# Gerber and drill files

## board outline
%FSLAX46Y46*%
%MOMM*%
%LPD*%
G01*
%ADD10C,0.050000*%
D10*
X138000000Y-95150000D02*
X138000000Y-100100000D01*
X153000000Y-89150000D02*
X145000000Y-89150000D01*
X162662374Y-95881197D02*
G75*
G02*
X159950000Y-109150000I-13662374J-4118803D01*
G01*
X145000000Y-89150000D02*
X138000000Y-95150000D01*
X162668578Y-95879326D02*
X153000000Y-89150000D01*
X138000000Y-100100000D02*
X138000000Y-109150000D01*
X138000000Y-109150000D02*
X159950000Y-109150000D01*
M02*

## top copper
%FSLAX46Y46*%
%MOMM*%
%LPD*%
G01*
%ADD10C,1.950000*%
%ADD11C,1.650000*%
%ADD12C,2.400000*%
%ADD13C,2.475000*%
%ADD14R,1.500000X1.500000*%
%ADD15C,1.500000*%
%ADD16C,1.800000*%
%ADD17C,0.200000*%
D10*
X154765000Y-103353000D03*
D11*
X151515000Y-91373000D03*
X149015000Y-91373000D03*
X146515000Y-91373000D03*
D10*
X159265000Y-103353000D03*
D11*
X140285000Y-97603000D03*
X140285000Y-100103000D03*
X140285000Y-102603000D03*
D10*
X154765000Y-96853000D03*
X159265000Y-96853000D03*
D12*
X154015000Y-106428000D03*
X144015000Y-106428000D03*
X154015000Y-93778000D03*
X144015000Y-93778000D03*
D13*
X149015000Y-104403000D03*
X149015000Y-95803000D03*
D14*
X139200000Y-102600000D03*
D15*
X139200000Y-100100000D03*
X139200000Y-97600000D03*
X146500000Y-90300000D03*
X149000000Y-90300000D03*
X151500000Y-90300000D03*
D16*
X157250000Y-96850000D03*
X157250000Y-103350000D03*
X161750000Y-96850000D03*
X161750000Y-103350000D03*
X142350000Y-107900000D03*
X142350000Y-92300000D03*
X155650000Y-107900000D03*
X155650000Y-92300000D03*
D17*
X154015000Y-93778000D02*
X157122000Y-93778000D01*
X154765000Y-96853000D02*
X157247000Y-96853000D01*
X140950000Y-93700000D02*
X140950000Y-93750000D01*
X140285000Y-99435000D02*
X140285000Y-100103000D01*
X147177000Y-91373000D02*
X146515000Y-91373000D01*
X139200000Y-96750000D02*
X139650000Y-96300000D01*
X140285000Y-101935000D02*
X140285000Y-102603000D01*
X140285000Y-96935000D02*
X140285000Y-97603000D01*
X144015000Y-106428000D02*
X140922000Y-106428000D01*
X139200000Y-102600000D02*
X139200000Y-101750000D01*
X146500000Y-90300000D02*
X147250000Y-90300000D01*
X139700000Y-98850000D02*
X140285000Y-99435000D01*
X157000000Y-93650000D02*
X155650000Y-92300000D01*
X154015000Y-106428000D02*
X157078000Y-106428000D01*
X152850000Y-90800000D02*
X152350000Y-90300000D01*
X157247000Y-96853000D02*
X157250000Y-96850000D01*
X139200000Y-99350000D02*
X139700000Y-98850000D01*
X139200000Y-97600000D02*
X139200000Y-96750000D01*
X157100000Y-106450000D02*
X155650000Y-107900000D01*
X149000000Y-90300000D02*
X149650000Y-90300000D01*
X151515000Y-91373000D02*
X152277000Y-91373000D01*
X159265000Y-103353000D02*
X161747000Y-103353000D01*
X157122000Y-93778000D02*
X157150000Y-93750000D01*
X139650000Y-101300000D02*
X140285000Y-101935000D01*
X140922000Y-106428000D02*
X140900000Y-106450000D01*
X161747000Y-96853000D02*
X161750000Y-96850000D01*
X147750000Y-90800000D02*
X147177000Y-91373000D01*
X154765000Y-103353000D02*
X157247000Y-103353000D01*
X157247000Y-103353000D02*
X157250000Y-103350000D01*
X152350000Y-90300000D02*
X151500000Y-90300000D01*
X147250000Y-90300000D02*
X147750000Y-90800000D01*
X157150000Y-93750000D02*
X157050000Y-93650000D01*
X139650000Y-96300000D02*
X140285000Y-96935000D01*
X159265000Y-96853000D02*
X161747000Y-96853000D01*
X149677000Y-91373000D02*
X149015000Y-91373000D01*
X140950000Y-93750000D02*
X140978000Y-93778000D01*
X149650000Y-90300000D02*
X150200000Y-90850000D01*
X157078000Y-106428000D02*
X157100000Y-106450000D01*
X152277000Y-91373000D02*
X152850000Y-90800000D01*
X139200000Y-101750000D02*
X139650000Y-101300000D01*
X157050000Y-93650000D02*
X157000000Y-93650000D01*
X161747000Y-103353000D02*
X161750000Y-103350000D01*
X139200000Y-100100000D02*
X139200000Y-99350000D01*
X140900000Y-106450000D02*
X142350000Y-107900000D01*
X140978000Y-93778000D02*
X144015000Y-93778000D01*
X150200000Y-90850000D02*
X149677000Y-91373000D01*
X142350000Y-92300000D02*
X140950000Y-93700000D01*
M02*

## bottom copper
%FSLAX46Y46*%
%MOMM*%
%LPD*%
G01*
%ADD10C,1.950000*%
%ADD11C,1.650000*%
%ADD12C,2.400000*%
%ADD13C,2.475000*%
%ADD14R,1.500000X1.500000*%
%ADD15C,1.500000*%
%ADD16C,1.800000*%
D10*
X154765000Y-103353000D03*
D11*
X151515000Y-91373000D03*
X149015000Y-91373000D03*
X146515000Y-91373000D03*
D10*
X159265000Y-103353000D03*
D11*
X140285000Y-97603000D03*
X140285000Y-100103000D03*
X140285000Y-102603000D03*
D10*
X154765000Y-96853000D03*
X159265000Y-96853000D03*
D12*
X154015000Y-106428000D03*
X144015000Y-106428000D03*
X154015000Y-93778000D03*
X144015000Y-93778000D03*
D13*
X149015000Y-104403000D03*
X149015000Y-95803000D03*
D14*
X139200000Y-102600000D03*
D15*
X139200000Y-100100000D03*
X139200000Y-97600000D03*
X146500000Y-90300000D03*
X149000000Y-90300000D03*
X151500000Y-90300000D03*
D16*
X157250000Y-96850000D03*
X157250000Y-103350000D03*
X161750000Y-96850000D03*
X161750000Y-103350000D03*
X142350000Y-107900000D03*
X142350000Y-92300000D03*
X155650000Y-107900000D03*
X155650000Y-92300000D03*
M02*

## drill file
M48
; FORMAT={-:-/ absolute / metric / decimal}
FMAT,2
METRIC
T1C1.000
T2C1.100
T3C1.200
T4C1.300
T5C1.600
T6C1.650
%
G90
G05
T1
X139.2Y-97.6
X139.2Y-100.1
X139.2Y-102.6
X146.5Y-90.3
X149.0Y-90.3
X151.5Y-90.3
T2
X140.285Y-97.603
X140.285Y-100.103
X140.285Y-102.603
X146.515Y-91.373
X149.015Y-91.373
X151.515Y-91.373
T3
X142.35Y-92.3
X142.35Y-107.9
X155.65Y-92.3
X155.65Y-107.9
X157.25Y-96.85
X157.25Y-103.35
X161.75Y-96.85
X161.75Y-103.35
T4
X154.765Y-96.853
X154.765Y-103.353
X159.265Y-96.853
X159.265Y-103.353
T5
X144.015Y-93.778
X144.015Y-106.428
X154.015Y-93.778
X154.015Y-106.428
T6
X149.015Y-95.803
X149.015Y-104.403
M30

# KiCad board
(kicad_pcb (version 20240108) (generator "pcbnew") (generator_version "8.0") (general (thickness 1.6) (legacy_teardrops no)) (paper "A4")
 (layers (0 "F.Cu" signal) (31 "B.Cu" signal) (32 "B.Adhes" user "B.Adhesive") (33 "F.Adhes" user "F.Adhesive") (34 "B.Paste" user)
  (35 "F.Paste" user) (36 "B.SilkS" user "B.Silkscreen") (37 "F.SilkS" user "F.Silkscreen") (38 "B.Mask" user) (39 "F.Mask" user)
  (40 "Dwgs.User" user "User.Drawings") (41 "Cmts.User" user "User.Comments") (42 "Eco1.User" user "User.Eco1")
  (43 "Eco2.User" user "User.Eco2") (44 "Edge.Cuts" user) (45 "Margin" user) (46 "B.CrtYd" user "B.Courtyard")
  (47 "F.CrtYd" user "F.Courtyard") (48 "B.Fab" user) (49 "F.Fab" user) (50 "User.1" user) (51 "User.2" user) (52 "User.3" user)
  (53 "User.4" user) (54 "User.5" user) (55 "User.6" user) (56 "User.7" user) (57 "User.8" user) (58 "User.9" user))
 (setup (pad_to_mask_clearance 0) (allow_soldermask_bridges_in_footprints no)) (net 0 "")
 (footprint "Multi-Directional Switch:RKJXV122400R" (layer "F.Cu") (at 149.2 98.5)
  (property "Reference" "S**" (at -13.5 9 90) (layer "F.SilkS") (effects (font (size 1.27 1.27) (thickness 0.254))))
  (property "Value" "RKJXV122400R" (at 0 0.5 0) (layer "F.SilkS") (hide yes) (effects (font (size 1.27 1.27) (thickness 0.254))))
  (pad "A1" thru_hole circle (at 5.565 4.853 90) (size 1.95 1.95) (drill 1.3) (layers "*.Cu" "*.Mask") (remove_unused_layers no))
  (pad "A11" thru_hole circle (at 2.315 -7.127 90) (size 1.65 1.65) (drill 1.1) (layers "*.Cu" "*.Mask") (remove_unused_layers no))
  (pad "A12" thru_hole circle (at -0.185 -7.127 90) (size 1.65 1.65) (drill 1.1) (layers "*.Cu" "*.Mask") (remove_unused_layers no))
  (pad "A13" thru_hole circle (at -2.685 -7.127 90) (size 1.65 1.65) (drill 1.1) (layers "*.Cu" "*.Mask") (remove_unused_layers no))
  (pad "B1" thru_hole circle (at 10.065 4.853 90) (size 1.95 1.95) (drill 1.3) (layers "*.Cu" "*.Mask") (remove_unused_layers no))
  (pad "B11" thru_hole circle (at -8.915 -0.897 90) (size 1.65 1.65) (drill 1.1) (layers "*.Cu" "*.Mask") (remove_unused_layers no))
  (pad "B12" thru_hole circle (at -8.915 1.603 90) (size 1.65 1.65) (drill 1.1) (layers "*.Cu" "*.Mask") (remove_unused_layers no))
  (pad "B13" thru_hole circle (at -8.915 4.103 90) (size 1.65 1.65) (drill 1.1) (layers "*.Cu" "*.Mask") (remove_unused_layers no))
  (pad "C1" thru_hole circle (at 5.565 -1.647 90) (size 1.95 1.95) (drill 1.3) (layers "*.Cu" "*.Mask") (remove_unused_layers no))
  (pad "D1" thru_hole circle (at 10.065 -1.647 90) (size 1.95 1.95) (drill 1.3) (layers "*.Cu" "*.Mask") (remove_unused_layers no))
  (pad "MH1" thru_hole circle (at 4.815 7.928 90) (size 2.4 2.4) (drill 1.6) (layers "*.Cu" "*.Mask") (remove_unused_layers no))
  (pad "MH2" thru_hole circle (at -5.185 7.928 90) (size 2.4 2.4) (drill 1.6) (layers "*.Cu" "*.Mask") (remove_unused_layers no))
  (pad "MH3" thru_hole circle (at 4.815 -4.722 90) (size 2.4 2.4) (drill 1.6) (layers "*.Cu" "*.Mask") (remove_unused_layers no))
  (pad "MH4" thru_hole circle (at -5.185 -4.722 90) (size 2.4 2.4) (drill 1.6) (layers "*.Cu" "*.Mask") (remove_unused_layers no))
  (pad "MH5" thru_hole circle (at -0.185 5.903 90) (size 2.475 2.475) (drill 1.65) (layers "*.Cu" "*.Mask") (remove_unused_layers no))
  (pad "MH6" thru_hole circle (at -0.185 -2.697 90) (size 2.475 2.475) (drill 1.65) (layers "*.Cu" "*.Mask") (remove_unused_layers no)))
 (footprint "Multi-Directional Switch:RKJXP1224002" (layer "F.Cu") (at 150 100)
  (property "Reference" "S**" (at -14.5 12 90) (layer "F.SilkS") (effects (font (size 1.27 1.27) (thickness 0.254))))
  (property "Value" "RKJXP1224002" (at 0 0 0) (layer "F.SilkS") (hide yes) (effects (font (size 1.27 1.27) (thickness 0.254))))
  (pad "1" thru_hole rect (at -10.8 2.6 90) (size 1.5 1.5) (drill 1) (layers "*.Cu" "*.Mask") (remove_unused_layers no))
  (pad "2" thru_hole circle (at -10.8 0.1 90) (size 1.5 1.5) (drill 1) (layers "*.Cu" "*.Mask") (remove_unused_layers no))
  (pad "3" thru_hole circle (at -10.8 -2.4 90) (size 1.5 1.5) (drill 1) (layers "*.Cu" "*.Mask") (remove_unused_layers no))
  (pad "4" thru_hole circle (at -3.5 -9.7 90) (size 1.5 1.5) (drill 1) (layers "*.Cu" "*.Mask") (remove_unused_layers no))
  (pad "5" thru_hole circle (at -1 -9.7 90) (size 1.5 1.5) (drill 1) (layers "*.Cu" "*.Mask") (remove_unused_layers no))
  (pad "6" thru_hole circle (at 1.5 -9.7 90) (size 1.5 1.5) (drill 1) (layers "*.Cu" "*.Mask") (remove_unused_layers no))
  (pad "7" thru_hole circle (at 7.25 -3.15 90) (size 1.8 1.8) (drill 1.2) (layers "*.Cu" "*.Mask") (remove_unused_layers no))
  (pad "8" thru_hole circle (at 7.25 3.35 90) (size 1.8 1.8) (drill 1.2) (layers "*.Cu" "*.Mask") (remove_unused_layers no))
  (pad "9" thru_hole circle (at 11.75 -3.15 90) (size 1.8 1.8) (drill 1.2) (layers "*.Cu" "*.Mask") (remove_unused_layers no))
  (pad "10" thru_hole circle (at 11.75 3.35 90) (size 1.8 1.8) (drill 1.2) (layers "*.Cu" "*.Mask") (remove_unused_layers no))
  (pad "MH1" thru_hole circle (at -7.65 7.9 90) (size 1.8 1.8) (drill 1.2) (layers "*.Cu" "*.Mask") (remove_unused_layers no))
  (pad "MH2" thru_hole circle (at -7.65 -7.7 90) (size 1.8 1.8) (drill 1.2) (layers "*.Cu" "*.Mask") (remove_unused_layers no))
  (pad "MH3" thru_hole circle (at 5.65 7.9 90) (size 1.8 1.8) (drill 1.2) (layers "*.Cu" "*.Mask") (remove_unused_layers no))
  (pad "MH4" thru_hole circle (at 5.65 -7.7 90) (size 1.8 1.8) (drill 1.2) (layers "*.Cu" "*.Mask") (remove_unused_layers no)))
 (gr_line (start 138 95.15) (end 138 100.1) (stroke (width 0.05) (type default)) (layer "Edge.Cuts"))
 (gr_line (start 153 89.15) (end 145 89.15) (stroke (width 0.05) (type default)) (layer "Edge.Cuts"))
 (gr_arc (start 162.662374 95.881197) (mid 162.980612 102.85788) (end 159.95 109.15) (stroke (width 0.05) (type default))
  (layer "Edge.Cuts"))
 (gr_line (start 145 89.15) (end 138 95.15) (stroke (width 0.05) (type default)) (layer "Edge.Cuts"))
 (gr_line (start 162.668578 95.879326) (end 153 89.15) (stroke (width 0.05) (type default)) (layer "Edge.Cuts"))
 (gr_line (start 138 100.1) (end 138 109.15) (stroke (width 0.05) (type default)) (layer "Edge.Cuts"))
 (gr_line (start 138 109.15) (end 159.95 109.15) (stroke (width 0.05) (type default)) (layer "Edge.Cuts"))
 (segment (start 154.015 93.778) (end 157.122 93.778) (width 0.2) (layer "F.Cu") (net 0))
 (segment (start 154.765 96.853) (end 157.247 96.853) (width 0.2) (layer "F.Cu") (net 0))
 (segment (start 140.95 93.7) (end 140.95 93.75) (width 0.2) (layer "F.Cu") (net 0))
 (segment (start 140.285 99.435) (end 140.285 100.103) (width 0.2) (layer "F.Cu") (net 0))
 (segment (start 147.177 91.373) (end 146.515 91.373) (width 0.2) (layer "F.Cu") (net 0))
 (segment (start 139.2 96.75) (end 139.65 96.3) (width 0.2) (layer "F.Cu") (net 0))
 (segment (start 140.285 101.935) (end 140.285 102.603) (width 0.2) (layer "F.Cu") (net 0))
 (segment (start 140.285 96.935) (end 140.285 97.603) (width 0.2) (layer "F.Cu") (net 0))
 (segment (start 144.015 106.428) (end 140.922 106.428) (width 0.2) (layer "F.Cu") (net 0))
 (segment (start 139.2 102.6) (end 139.2 101.75) (width 0.2) (layer "F.Cu") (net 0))
 (segment (start 146.5 90.3) (end 147.25 90.3) (width 0.2) (layer "F.Cu") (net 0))
 (segment (start 139.7 98.85) (end 140.285 99.435) (width 0.2) (layer "F.Cu") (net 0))
 (segment (start 157 93.65) (end 155.65 92.3) (width 0.2) (layer "F.Cu") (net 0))
 (segment (start 154.015 106.428) (end 157.078 106.428) (width 0.2) (layer "F.Cu") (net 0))
 (segment (start 152.85 90.8) (end 152.35 90.3) (width 0.2) (layer "F.Cu") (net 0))
 (segment (start 157.247 96.853) (end 157.25 96.85) (width 0.2) (layer "F.Cu") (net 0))
 (segment (start 139.2 99.35) (end 139.7 98.85) (width 0.2) (layer "F.Cu") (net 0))
 (segment (start 139.2 97.6) (end 139.2 96.75) (width 0.2) (layer "F.Cu") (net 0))
 (segment (start 157.1 106.45) (end 155.65 107.9) (width 0.2) (layer "F.Cu") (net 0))
 (segment (start 149 90.3) (end 149.65 90.3) (width 0.2) (layer "F.Cu") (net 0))
 (segment (start 151.515 91.373) (end 152.277 91.373) (width 0.2) (layer "F.Cu") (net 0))
 (segment (start 159.265 103.353) (end 161.747 103.353) (width 0.2) (layer "F.Cu") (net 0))
 (segment (start 157.122 93.778) (end 157.15 93.75) (width 0.2) (layer "F.Cu") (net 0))
 (segment (start 139.65 101.3) (end 140.285 101.935) (width 0.2) (layer "F.Cu") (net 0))
 (segment (start 140.922 106.428) (end 140.9 106.45) (width 0.2) (layer "F.Cu") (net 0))
 (segment (start 161.747 96.853) (end 161.75 96.85) (width 0.2) (layer "F.Cu") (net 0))
 (segment (start 147.75 90.8) (end 147.177 91.373) (width 0.2) (layer "F.Cu") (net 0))
 (segment (start 154.765 103.353) (end 157.247 103.353) (width 0.2) (layer "F.Cu") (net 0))
 (segment (start 157.247 103.353) (end 157.25 103.35) (width 0.2) (layer "F.Cu") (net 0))
 (segment (start 152.35 90.3) (end 151.5 90.3) (width 0.2) (layer "F.Cu") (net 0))
 (segment (start 147.25 90.3) (end 147.75 90.8) (width 0.2) (layer "F.Cu") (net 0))
 (segment (start 157.15 93.75) (end 157.05 93.65) (width 0.2) (layer "F.Cu") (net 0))
 (segment (start 139.65 96.3) (end 140.285 96.935) (width 0.2) (layer "F.Cu") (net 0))
 (segment (start 159.265 96.853) (end 161.747 96.853) (width 0.2) (layer "F.Cu") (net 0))
 (segment (start 149.677 91.373) (end 149.015 91.373) (width 0.2) (layer "F.Cu") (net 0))
 (segment (start 140.95 93.75) (end 140.978 93.778) (width 0.2) (layer "F.Cu") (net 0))
 (segment (start 149.65 90.3) (end 150.2 90.85) (width 0.2) (layer "F.Cu") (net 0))
 (segment (start 157.078 106.428) (end 157.1 106.45) (width 0.2) (layer "F.Cu") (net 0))
 (segment (start 152.277 91.373) (end 152.85 90.8) (width 0.2) (layer "F.Cu") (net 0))
 (segment (start 139.2 101.75) (end 139.65 101.3) (width 0.2) (layer "F.Cu") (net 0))
 (segment (start 157.05 93.65) (end 157 93.65) (width 0.2) (layer "F.Cu") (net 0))
 (segment (start 161.747 103.353) (end 161.75 103.35) (width 0.2) (layer "F.Cu") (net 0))
 (segment (start 139.2 100.1) (end 139.2 99.35) (width 0.2) (layer "F.Cu") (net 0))
 (segment (start 140.9 106.45) (end 142.35 107.9) (width 0.2) (layer "F.Cu") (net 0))
 (segment (start 140.978 93.778) (end 144.015 93.778) (width 0.2) (layer "F.Cu") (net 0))
 (segment (start 150.2 90.85) (end 149.677 91.373) (width 0.2) (layer "F.Cu") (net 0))
 (segment (start 142.35 92.3) (end 140.95 93.7) (width 0.2) (layer "F.Cu") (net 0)))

